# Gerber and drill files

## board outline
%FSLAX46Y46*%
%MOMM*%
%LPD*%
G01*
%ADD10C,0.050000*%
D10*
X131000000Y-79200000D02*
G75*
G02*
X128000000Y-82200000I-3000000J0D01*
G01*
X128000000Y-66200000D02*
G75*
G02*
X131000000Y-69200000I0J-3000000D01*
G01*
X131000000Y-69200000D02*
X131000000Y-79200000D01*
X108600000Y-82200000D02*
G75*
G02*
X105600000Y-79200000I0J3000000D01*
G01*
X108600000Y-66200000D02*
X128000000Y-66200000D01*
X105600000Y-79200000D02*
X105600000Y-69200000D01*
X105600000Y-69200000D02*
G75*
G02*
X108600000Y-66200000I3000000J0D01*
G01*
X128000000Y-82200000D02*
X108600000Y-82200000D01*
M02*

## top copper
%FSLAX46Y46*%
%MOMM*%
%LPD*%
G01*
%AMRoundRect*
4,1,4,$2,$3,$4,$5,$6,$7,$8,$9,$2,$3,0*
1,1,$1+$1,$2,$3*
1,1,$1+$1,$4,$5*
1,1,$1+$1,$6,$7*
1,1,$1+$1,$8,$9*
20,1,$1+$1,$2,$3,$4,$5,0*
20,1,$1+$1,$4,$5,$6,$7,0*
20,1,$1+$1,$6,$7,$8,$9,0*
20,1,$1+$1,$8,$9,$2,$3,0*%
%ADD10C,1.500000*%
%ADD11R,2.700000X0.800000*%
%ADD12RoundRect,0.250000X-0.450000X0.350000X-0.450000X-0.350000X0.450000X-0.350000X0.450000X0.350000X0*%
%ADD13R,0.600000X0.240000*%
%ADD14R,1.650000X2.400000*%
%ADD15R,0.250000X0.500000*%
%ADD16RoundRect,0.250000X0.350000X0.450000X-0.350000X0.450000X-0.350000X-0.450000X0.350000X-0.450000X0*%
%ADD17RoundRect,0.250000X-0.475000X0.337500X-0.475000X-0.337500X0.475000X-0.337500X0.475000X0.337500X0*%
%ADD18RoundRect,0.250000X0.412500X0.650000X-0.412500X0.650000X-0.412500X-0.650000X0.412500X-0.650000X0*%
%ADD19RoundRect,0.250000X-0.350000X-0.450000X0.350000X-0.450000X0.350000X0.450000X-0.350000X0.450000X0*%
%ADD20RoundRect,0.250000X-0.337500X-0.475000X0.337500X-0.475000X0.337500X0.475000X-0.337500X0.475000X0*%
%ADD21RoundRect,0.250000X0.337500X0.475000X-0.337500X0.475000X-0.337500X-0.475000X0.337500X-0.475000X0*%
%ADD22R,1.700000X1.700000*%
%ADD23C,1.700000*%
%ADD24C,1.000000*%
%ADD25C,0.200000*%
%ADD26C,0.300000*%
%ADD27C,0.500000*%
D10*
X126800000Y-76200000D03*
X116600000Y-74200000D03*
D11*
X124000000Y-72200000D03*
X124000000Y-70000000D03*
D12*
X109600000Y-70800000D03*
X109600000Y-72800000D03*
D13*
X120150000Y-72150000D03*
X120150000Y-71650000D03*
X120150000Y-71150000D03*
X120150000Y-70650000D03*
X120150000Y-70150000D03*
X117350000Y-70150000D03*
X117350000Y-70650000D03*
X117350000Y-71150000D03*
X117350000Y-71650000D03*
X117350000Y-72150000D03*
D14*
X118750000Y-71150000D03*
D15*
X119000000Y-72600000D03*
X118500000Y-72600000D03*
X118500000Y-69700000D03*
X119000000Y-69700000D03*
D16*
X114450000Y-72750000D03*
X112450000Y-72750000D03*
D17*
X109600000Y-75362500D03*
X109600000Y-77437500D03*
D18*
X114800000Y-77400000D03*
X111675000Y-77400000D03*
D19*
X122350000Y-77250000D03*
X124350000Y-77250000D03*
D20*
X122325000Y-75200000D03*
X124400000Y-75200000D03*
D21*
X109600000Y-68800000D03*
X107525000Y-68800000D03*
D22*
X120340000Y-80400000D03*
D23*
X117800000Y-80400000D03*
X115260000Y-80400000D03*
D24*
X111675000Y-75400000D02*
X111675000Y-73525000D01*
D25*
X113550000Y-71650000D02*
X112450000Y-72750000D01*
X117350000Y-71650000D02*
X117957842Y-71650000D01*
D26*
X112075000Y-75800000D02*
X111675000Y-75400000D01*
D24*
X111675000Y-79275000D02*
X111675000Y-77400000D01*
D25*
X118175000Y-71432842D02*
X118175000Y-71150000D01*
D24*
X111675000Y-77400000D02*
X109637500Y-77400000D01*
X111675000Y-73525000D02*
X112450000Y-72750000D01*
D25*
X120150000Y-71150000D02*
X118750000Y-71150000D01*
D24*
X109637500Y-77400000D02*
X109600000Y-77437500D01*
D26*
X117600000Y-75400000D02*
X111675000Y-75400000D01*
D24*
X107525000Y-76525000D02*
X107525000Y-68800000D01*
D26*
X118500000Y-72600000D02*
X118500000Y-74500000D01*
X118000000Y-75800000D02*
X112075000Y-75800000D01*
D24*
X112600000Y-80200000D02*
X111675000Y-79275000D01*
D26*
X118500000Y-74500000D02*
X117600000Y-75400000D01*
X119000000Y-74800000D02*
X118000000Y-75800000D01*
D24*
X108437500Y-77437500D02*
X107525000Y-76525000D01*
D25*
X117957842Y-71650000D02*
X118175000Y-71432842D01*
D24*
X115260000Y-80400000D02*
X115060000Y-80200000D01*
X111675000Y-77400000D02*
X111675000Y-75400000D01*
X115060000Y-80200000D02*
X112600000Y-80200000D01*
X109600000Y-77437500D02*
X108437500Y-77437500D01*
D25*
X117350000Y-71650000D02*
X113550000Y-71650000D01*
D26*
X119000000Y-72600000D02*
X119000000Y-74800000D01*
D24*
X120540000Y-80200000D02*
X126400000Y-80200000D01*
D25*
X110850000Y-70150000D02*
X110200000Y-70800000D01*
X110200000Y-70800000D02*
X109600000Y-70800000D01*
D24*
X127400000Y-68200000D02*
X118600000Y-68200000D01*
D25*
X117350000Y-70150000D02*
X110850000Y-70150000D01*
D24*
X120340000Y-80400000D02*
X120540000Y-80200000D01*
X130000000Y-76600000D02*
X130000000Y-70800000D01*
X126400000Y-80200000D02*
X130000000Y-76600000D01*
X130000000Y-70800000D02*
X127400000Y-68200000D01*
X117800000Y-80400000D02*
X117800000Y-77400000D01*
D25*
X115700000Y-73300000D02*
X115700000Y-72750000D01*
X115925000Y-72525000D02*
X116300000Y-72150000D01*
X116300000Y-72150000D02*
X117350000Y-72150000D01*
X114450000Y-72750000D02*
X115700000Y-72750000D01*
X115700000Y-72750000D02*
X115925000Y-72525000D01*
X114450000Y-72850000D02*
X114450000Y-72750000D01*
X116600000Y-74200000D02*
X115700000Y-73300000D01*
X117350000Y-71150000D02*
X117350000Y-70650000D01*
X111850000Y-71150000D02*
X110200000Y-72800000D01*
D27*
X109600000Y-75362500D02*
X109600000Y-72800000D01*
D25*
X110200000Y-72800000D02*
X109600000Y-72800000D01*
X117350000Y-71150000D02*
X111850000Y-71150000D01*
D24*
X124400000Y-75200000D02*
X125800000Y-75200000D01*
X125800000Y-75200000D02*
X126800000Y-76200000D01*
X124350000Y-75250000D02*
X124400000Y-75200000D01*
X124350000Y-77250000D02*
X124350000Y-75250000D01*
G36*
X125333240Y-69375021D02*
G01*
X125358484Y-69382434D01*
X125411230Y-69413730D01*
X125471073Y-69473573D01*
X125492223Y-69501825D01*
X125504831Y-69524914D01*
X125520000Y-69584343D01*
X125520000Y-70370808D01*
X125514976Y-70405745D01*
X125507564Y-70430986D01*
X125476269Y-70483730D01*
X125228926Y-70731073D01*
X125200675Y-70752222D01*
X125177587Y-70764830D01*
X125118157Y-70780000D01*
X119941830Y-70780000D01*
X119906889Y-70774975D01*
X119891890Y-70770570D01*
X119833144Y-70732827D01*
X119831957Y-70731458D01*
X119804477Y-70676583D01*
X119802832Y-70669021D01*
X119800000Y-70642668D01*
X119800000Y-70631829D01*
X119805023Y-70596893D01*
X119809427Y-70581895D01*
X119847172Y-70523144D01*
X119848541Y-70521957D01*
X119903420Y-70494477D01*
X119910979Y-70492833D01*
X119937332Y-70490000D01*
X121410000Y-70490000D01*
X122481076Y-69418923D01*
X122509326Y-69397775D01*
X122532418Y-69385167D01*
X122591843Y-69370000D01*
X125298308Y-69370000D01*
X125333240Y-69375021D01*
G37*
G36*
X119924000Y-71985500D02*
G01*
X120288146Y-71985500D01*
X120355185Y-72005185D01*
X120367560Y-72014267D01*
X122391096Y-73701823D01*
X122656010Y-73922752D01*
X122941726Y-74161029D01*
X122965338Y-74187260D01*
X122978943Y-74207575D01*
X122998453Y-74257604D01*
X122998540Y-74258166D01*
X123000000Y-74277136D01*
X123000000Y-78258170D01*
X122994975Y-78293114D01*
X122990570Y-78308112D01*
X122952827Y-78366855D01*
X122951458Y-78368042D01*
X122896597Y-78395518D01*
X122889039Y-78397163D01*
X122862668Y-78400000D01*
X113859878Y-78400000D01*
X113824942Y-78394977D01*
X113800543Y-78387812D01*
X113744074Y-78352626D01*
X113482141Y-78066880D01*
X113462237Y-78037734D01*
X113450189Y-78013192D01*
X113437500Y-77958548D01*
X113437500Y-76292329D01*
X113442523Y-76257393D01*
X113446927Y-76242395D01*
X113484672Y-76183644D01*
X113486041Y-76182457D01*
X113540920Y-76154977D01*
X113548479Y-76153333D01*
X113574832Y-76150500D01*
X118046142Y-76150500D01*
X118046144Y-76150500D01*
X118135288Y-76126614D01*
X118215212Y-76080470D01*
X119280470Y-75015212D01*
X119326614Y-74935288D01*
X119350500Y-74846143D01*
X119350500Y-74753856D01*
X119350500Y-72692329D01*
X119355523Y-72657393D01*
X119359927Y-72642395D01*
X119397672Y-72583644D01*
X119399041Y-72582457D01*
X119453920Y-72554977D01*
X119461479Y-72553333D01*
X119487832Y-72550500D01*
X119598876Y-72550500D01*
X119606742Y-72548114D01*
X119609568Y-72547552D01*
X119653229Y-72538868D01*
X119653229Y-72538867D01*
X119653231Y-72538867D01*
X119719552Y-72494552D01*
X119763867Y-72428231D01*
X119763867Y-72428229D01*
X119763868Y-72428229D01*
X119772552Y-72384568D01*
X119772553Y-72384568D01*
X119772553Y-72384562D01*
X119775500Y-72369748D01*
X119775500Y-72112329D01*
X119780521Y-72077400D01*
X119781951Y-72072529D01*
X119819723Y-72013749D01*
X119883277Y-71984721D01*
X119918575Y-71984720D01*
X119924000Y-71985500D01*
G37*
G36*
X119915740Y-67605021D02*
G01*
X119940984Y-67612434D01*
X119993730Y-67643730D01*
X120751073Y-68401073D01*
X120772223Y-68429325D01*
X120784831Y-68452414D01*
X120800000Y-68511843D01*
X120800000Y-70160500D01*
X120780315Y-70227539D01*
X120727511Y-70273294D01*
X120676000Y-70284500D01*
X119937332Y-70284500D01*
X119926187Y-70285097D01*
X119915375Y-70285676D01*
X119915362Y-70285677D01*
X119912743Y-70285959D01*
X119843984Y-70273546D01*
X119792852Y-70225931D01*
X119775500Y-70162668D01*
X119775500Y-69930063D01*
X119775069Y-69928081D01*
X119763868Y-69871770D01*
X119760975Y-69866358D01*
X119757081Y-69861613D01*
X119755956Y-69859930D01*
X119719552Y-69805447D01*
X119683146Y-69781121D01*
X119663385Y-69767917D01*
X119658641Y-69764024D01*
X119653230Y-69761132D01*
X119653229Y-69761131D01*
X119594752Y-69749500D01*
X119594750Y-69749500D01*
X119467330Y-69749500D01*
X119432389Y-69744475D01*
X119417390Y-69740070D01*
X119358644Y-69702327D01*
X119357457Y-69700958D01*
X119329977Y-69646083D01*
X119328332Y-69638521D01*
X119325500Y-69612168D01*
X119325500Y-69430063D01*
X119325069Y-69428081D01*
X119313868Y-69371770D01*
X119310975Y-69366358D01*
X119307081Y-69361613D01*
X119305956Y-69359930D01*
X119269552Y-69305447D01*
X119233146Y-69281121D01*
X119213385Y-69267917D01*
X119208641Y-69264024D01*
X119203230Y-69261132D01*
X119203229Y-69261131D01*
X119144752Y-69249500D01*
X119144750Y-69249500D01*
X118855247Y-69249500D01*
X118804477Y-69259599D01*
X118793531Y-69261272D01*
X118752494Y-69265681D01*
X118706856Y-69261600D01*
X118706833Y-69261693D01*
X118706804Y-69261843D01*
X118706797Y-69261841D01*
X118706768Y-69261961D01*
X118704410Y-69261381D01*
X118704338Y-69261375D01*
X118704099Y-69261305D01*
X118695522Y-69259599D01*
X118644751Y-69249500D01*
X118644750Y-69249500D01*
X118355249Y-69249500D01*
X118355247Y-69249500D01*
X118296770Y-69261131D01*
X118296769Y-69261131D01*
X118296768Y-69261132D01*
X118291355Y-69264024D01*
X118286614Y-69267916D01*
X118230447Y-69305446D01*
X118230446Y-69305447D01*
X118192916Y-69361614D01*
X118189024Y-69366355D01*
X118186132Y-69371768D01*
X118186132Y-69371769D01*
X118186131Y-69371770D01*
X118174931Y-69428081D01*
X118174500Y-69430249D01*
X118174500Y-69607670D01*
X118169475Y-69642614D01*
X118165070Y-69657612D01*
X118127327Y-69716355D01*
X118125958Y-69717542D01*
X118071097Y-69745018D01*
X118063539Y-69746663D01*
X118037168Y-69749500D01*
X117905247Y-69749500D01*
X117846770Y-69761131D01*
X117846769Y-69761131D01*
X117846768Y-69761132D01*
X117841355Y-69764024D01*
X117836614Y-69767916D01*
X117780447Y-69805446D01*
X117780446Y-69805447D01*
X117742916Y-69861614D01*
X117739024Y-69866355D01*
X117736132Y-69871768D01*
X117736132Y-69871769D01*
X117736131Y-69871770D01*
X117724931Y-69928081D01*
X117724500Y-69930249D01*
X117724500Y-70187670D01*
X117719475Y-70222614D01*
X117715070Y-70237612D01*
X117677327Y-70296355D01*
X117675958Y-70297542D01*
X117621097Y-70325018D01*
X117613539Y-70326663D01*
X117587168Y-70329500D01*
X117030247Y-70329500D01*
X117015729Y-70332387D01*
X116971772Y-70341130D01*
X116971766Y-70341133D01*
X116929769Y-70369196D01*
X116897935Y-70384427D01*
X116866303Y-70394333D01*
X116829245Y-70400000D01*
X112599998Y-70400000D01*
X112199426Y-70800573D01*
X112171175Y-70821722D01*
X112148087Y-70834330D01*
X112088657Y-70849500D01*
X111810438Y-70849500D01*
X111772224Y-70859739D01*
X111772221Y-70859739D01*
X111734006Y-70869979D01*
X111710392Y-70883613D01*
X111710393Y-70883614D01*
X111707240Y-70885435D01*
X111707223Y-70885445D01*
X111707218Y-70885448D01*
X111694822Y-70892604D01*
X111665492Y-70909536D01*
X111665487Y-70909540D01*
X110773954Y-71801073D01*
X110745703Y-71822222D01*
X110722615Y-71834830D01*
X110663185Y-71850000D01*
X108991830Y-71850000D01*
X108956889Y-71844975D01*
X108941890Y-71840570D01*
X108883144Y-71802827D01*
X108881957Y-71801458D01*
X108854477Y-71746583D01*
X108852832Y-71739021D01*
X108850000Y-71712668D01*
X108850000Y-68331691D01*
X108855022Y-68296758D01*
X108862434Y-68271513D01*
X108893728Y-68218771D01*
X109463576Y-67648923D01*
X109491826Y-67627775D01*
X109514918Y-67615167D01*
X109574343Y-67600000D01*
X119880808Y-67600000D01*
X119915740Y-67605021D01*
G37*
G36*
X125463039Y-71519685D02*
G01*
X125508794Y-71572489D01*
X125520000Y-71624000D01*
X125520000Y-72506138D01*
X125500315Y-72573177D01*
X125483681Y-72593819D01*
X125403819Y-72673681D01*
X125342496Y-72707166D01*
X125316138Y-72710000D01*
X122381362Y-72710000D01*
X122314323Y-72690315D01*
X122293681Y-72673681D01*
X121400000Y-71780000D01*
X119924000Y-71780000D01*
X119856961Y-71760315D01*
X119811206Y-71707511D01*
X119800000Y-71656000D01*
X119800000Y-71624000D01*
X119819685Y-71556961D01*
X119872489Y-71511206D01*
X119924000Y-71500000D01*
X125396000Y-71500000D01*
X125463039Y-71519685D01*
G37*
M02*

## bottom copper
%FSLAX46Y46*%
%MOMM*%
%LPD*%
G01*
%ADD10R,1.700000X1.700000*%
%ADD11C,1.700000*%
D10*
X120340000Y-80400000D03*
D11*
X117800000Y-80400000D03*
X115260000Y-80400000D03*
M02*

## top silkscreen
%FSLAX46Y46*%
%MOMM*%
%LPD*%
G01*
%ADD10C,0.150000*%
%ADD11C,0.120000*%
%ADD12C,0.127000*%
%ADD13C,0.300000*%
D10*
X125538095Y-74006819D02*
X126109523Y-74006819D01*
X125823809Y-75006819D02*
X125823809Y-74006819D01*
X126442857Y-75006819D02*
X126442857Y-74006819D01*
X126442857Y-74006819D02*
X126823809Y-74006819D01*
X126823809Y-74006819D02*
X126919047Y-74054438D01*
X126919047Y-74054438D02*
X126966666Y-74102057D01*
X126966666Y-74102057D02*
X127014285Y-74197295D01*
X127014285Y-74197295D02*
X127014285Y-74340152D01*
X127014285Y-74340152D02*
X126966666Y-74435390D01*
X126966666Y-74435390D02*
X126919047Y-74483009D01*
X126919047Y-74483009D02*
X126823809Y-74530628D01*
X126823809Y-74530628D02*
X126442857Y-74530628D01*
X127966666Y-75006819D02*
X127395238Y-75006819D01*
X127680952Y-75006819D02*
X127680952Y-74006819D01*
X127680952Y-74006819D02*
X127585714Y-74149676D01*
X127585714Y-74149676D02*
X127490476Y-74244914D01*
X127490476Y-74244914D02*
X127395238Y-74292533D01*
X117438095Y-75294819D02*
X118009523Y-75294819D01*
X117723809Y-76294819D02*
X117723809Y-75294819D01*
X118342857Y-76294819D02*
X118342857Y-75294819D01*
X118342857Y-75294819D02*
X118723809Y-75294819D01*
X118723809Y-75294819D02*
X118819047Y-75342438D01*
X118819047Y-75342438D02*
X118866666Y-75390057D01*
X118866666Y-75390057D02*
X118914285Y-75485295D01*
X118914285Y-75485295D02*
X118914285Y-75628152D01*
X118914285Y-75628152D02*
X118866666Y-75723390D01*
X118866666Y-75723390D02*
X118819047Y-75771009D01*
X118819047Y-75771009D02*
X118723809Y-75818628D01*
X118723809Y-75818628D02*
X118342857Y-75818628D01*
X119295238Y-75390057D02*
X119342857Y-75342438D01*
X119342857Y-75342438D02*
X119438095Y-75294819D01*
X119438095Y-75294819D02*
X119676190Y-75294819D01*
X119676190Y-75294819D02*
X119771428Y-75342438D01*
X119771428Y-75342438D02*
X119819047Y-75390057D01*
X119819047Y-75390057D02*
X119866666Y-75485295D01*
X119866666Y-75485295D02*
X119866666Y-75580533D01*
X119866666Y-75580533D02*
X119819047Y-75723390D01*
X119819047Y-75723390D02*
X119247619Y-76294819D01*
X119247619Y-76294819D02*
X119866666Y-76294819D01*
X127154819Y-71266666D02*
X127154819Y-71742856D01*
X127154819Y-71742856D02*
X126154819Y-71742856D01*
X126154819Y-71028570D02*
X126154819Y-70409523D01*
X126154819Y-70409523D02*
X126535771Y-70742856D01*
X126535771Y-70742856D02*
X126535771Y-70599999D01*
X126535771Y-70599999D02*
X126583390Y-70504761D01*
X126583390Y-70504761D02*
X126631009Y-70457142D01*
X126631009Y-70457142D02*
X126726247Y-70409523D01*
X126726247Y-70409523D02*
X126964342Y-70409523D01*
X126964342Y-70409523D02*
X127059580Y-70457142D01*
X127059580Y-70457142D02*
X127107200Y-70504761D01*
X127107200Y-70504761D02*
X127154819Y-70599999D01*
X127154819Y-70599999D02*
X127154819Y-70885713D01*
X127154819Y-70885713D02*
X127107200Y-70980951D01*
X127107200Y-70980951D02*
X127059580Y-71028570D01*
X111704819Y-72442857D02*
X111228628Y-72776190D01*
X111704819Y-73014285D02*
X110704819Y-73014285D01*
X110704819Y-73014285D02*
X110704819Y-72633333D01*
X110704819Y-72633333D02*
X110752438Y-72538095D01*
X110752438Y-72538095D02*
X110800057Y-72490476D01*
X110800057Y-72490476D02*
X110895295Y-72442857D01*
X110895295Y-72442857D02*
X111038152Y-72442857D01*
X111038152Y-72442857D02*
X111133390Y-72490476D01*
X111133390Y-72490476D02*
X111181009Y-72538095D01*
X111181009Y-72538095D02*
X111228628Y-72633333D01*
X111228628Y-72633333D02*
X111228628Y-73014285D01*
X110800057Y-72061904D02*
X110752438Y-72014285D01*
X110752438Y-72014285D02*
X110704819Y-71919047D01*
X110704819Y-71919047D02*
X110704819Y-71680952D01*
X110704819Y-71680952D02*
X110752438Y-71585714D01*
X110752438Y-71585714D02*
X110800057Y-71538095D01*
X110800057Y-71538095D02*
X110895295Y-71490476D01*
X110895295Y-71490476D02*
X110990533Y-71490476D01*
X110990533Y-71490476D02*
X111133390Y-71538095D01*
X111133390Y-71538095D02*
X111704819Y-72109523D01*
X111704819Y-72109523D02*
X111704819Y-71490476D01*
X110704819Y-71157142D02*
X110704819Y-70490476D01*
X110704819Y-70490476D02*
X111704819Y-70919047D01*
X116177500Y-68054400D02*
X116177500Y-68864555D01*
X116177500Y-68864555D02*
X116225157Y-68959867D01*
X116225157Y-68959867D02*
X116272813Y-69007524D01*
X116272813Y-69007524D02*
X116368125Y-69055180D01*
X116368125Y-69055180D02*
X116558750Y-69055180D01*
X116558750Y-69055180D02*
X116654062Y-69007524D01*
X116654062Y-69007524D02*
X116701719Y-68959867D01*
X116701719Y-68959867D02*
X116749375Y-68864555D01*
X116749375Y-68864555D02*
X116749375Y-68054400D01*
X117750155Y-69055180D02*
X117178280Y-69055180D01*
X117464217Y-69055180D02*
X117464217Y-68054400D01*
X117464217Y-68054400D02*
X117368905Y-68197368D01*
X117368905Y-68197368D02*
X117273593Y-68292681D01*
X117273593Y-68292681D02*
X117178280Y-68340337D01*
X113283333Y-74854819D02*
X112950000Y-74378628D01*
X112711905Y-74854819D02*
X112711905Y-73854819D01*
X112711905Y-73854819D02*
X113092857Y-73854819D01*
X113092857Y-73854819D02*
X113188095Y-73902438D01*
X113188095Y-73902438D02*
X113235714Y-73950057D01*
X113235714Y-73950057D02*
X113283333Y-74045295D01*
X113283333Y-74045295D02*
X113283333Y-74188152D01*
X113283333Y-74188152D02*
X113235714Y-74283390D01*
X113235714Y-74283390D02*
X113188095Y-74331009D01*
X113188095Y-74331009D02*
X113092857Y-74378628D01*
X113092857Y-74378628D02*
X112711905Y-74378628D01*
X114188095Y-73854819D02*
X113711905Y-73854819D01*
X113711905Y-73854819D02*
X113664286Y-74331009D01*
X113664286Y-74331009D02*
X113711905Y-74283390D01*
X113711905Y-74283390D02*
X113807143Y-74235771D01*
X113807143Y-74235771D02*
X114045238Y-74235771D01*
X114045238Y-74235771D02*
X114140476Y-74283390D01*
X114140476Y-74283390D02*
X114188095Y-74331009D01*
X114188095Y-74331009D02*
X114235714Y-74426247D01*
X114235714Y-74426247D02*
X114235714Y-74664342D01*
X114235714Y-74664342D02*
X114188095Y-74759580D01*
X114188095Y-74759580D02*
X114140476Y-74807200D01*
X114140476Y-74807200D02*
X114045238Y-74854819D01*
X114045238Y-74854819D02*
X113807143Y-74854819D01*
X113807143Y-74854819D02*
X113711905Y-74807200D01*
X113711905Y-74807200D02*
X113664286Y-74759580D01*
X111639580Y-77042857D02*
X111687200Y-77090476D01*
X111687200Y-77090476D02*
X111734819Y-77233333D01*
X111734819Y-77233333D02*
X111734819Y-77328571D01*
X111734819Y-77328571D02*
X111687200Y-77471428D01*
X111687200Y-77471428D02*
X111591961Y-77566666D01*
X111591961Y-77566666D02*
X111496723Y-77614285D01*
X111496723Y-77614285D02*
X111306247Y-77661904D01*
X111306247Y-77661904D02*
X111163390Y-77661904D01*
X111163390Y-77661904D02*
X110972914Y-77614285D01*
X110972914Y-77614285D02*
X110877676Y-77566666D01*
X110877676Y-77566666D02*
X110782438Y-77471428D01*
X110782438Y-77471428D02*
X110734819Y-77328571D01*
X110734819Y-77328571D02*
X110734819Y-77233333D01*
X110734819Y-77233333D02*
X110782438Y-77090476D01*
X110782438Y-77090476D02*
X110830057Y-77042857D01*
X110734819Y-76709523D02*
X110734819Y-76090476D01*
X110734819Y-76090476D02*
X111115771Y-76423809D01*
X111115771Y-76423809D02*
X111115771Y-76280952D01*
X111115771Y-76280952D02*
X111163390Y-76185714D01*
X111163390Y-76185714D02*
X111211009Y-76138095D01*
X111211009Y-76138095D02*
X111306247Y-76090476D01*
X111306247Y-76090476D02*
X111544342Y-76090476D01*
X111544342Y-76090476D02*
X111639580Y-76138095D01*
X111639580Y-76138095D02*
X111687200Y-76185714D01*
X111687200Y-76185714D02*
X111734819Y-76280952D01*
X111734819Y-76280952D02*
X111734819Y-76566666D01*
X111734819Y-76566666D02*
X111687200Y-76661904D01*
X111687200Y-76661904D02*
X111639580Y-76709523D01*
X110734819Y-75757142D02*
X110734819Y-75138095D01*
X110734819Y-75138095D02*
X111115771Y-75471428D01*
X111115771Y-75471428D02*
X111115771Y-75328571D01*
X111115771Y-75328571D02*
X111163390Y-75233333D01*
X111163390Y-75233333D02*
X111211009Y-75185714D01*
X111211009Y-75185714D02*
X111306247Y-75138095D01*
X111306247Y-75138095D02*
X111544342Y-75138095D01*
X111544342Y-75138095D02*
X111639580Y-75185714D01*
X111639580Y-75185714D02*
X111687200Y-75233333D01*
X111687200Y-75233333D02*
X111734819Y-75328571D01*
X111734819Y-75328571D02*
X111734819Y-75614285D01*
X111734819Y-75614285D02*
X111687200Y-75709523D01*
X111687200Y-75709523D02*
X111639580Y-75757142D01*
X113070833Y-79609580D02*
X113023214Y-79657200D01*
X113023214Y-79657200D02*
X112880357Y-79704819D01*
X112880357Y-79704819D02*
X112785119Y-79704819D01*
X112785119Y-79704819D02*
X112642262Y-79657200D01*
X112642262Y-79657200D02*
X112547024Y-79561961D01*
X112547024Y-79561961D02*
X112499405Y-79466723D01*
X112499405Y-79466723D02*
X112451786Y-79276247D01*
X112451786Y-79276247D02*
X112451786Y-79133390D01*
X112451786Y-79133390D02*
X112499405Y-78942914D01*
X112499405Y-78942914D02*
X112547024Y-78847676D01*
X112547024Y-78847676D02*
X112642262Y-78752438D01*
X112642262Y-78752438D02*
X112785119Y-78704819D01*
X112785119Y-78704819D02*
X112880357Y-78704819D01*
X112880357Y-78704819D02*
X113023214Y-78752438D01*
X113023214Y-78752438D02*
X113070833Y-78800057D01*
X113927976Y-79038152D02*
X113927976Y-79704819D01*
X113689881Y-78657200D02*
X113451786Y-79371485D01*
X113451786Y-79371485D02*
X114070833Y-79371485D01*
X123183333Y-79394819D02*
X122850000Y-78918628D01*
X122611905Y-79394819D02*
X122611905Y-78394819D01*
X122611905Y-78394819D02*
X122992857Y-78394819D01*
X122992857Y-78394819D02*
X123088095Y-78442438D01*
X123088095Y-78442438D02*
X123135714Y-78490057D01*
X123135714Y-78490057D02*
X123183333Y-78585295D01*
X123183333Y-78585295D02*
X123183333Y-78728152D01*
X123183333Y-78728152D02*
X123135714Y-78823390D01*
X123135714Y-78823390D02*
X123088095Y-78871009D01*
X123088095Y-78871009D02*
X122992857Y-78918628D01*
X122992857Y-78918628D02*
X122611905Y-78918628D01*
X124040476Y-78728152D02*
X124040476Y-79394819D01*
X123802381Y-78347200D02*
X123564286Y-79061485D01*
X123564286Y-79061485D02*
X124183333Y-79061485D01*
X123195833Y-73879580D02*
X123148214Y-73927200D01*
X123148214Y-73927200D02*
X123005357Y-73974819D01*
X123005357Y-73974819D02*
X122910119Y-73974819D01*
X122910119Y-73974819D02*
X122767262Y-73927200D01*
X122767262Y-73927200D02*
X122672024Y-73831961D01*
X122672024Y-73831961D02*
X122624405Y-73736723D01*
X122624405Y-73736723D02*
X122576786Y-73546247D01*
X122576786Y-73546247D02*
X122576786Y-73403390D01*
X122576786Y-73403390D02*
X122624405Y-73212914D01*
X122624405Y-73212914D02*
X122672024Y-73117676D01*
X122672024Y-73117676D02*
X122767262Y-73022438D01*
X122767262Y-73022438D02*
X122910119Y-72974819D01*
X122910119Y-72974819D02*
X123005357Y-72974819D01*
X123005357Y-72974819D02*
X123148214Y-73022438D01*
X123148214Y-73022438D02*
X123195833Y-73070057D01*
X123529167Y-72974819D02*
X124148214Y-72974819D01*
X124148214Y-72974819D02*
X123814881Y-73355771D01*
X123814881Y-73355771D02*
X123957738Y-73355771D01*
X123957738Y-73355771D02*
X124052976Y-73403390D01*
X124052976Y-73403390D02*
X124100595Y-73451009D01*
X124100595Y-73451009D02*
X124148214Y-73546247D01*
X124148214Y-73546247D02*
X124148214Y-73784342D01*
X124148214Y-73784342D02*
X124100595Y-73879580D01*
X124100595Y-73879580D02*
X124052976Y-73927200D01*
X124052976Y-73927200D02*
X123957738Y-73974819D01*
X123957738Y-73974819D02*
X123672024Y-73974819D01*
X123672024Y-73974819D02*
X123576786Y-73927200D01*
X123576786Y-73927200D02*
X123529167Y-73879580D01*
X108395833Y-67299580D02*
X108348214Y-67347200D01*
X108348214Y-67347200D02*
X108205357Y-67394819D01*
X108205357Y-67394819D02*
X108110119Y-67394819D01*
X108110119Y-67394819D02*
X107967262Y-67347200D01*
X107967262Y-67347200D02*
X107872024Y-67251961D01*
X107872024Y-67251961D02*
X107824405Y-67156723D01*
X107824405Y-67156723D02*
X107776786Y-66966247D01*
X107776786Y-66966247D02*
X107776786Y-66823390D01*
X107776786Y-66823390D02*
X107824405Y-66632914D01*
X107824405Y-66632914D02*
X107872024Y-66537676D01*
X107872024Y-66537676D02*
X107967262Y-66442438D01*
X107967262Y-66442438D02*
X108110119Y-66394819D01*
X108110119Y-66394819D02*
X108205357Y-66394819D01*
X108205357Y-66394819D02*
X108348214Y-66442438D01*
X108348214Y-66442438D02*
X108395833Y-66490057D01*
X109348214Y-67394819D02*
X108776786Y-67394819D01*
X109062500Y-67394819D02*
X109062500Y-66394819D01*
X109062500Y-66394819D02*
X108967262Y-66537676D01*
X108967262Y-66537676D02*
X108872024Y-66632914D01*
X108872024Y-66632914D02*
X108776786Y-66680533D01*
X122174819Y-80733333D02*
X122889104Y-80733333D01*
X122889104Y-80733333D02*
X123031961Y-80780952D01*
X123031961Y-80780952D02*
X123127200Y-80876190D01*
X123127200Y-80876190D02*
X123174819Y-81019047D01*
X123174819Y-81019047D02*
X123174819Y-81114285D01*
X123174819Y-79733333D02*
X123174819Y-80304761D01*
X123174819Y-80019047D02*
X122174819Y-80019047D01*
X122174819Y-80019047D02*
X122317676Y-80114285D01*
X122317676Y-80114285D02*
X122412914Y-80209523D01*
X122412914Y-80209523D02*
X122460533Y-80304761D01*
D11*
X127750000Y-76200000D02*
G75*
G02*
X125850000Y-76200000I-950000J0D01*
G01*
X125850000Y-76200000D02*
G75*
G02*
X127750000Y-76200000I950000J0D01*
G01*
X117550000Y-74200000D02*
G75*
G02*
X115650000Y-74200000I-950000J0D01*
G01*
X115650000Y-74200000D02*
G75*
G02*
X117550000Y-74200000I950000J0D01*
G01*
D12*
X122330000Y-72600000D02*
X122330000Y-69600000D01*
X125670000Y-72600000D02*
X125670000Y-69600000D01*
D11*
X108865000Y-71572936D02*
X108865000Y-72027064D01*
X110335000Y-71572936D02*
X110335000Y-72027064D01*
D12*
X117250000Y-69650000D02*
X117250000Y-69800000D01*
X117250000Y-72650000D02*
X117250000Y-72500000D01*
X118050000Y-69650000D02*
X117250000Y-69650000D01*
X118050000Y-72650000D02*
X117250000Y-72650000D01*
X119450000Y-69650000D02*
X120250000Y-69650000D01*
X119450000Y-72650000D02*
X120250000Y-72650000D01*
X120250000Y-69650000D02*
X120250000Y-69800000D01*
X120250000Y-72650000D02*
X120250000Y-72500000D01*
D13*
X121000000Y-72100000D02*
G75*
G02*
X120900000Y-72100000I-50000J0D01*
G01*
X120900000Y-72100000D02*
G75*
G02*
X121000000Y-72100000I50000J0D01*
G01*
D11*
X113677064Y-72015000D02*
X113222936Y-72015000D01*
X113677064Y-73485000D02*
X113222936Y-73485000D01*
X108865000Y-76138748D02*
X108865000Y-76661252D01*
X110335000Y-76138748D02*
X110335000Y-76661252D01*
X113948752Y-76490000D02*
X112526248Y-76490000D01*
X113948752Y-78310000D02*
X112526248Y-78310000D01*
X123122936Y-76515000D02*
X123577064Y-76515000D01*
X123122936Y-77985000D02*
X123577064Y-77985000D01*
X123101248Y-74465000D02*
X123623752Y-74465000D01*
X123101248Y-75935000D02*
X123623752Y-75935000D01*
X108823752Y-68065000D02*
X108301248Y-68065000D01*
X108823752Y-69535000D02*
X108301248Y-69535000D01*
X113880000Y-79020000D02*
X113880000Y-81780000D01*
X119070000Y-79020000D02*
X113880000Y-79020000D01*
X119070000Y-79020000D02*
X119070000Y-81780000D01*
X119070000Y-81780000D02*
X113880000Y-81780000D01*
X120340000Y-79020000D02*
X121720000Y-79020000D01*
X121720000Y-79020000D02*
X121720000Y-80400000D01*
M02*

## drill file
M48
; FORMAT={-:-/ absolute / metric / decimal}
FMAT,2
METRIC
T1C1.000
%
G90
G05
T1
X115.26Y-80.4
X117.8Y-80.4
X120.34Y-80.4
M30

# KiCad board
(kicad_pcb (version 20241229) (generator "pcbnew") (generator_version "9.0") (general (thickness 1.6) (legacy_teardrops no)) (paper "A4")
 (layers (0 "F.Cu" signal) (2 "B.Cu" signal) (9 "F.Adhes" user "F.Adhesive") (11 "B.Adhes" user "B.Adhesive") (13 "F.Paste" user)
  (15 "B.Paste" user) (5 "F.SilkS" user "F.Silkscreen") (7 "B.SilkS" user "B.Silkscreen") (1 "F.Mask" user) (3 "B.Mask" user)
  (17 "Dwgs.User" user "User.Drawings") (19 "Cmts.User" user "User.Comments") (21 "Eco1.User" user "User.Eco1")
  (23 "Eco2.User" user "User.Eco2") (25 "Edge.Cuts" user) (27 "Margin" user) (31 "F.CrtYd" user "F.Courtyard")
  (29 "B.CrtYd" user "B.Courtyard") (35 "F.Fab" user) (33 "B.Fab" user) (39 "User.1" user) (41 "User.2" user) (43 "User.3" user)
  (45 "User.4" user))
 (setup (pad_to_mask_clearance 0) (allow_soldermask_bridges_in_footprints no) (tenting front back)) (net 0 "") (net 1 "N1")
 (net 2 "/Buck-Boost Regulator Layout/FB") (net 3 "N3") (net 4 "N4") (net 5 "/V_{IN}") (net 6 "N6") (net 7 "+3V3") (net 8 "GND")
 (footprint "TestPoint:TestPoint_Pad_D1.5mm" (layer "F.Cu") (at 126.8 76.2)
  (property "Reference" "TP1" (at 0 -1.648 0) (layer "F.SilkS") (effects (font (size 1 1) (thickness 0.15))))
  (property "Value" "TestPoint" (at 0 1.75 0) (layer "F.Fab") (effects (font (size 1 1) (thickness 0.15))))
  (fp_circle (center 0 0) (end 0 0.95) (stroke (width 0.12) (type solid)) (fill no) (layer "F.SilkS"))
  (pad "1" smd circle (at 0 0) (size 1.5 1.5) (layers "F.Cu" "F.Mask") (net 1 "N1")))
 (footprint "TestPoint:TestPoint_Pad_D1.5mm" (layer "F.Cu") (at 116.6 74.2)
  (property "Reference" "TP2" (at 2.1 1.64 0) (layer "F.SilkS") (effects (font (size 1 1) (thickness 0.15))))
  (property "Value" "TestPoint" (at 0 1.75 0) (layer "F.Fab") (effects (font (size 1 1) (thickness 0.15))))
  (fp_circle (center 0 0) (end 0 0.95) (stroke (width 0.12) (type solid)) (fill no) (layer "F.SilkS"))
  (pad "1" smd circle (at 0 0) (size 1.5 1.5) (layers "F.Cu" "F.Mask") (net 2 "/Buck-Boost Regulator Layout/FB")))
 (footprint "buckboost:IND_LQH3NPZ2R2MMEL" (layer "F.Cu") (at 124 71.1 90)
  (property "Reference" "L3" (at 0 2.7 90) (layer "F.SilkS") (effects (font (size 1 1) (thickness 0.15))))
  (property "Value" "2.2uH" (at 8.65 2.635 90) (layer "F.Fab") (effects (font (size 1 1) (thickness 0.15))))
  (fp_line (start -1.5 -1.67) (end 1.5 -1.67) (stroke (width 0.127) (type solid)) (layer "F.SilkS"))
  (fp_line (start -1.5 1.67) (end 1.5 1.67) (stroke (width 0.127) (type solid)) (layer "F.SilkS"))
  (pad "1" smd rect (at -1.1 0 90) (size 0.8 2.7) (layers "F.Cu" "F.Mask" "F.Paste") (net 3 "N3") (solder_mask_margin 0.102))
  (pad "2" smd rect (at 1.1 0 90) (size 0.8 2.7) (layers "F.Cu" "F.Mask" "F.Paste") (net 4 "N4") (solder_mask_margin 0.102)))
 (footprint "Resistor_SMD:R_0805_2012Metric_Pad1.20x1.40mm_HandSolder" (layer "F.Cu") (at 109.6 71.8 -90)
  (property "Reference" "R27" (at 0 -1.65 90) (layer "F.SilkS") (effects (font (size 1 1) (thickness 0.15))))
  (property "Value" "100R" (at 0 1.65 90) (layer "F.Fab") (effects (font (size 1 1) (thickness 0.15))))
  (fp_line (start -0.227064 0.735) (end 0.227064 0.735) (stroke (width 0.12) (type solid)) (layer "F.SilkS"))
  (fp_line (start -0.227064 -0.735) (end 0.227064 -0.735) (stroke (width 0.12) (type solid)) (layer "F.SilkS"))
  (pad "1" smd roundrect (at -1 0 270) (size 1.2 1.4) (layers "F.Cu" "F.Mask" "F.Paste") (roundrect_rratio 0.208333) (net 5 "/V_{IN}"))
  (pad "2" smd roundrect (at 1 0 270) (size 1.2 1.4) (layers "F.Cu" "F.Mask" "F.Paste") (roundrect_rratio 0.208333) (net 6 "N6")))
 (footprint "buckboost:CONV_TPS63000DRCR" (layer "F.Cu") (at 118.75 71.15 180)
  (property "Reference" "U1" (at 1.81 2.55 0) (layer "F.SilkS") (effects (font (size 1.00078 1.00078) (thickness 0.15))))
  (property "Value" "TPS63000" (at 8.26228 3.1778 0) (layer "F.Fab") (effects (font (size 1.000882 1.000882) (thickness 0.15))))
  (fp_line (start 1.5 1.5) (end 1.5 1.35) (stroke (width 0.127) (type solid)) (layer "F.SilkS"))
  (fp_line (start 1.5 -1.5) (end 1.5 -1.35) (stroke (width 0.127) (type solid)) (layer "F.SilkS"))
  (fp_line (start 0.7 1.5) (end 1.5 1.5) (stroke (width 0.127) (type solid)) (layer "F.SilkS"))
  (fp_line (start 0.7 -1.5) (end 1.5 -1.5) (stroke (width 0.127) (type solid)) (layer "F.SilkS"))
  (fp_line (start -0.7 1.5) (end -1.5 1.5) (stroke (width 0.127) (type solid)) (layer "F.SilkS"))
  (fp_line (start -0.7 -1.5) (end -1.5 -1.5) (stroke (width 0.127) (type solid)) (layer "F.SilkS"))
  (fp_line (start -1.5 1.5) (end -1.5 1.35) (stroke (width 0.127) (type solid)) (layer "F.SilkS"))
  (fp_line (start -1.5 -1.5) (end -1.5 -1.35) (stroke (width 0.127) (type solid)) (layer "F.SilkS"))
  (fp_circle (center -2.2 -0.95) (end -2.15 -0.95) (stroke (width 0.3) (type solid)) (fill no) (layer "F.SilkS"))
  (pad "1" smd rect (at -1.4 -1 180) (size 0.6 0.24) (layers "F.Cu" "F.Mask" "F.Paste") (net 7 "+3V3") (solder_mask_margin 0.102))
  (pad "2" smd rect (at -1.4 -0.5 180) (size 0.6 0.24) (layers "F.Cu" "F.Mask" "F.Paste") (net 3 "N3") (solder_mask_margin 0.102))
  (pad "3" smd rect (at -1.4 0 180) (size 0.6 0.24) (layers "F.Cu" "F.Mask" "F.Paste") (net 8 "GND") (solder_mask_margin 0.102))
  (pad "4" smd rect (at -1.4 0.5 180) (size 0.6 0.24) (layers "F.Cu" "F.Mask" "F.Paste") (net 4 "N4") (solder_mask_margin 0.102))
  (pad "5" smd rect (at -1.4 1 180) (size 0.6 0.24) (layers "F.Cu" "F.Mask" "F.Paste") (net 5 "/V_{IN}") (solder_mask_margin 0.102))
  (pad "6" smd rect (at 1.4 1 180) (size 0.6 0.24) (layers "F.Cu" "F.Mask" "F.Paste") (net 5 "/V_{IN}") (solder_mask_margin 0.102))
  (pad "7" smd rect (at 1.4 0.5 180) (size 0.6 0.24) (layers "F.Cu" "F.Mask" "F.Paste") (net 6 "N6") (solder_mask_margin 0.102))
  (pad "8" smd rect (at 1.4 0 180) (size 0.6 0.24) (layers "F.Cu" "F.Mask" "F.Paste") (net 6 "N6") (solder_mask_margin 0.102))
  (pad "9" smd rect (at 1.4 -0.5 180) (size 0.6 0.24) (layers "F.Cu" "F.Mask" "F.Paste") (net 8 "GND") (solder_mask_margin 0.102))
  (pad "10" smd rect (at 1.4 -1 180) (size 0.6 0.24) (layers "F.Cu" "F.Mask" "F.Paste") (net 2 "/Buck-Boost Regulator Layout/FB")
   (solder_mask_margin 0.102))
  (pad "11" smd rect (at 0 0 180) (size 1.65 2.4) (layers "F.Cu" "F.Mask") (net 8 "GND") (solder_mask_margin 0.102))
  (pad "11_1" smd rect (at -0.25 -1.45 180) (size 0.25 0.5) (layers "F.Cu" "F.Mask") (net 8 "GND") (solder_mask_margin 0.102))
  (pad "11_2" smd rect (at 0.25 -1.45 180) (size 0.25 0.5) (layers "F.Cu" "F.Mask") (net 8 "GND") (solder_mask_margin 0.102))
  (pad "11_3" smd rect (at 0.25 1.45 180) (size 0.25 0.5) (layers "F.Cu" "F.Mask") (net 8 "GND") (solder_mask_margin 0.102))
  (pad "11_4" smd rect (at -0.25 1.45 180) (size 0.25 0.5) (layers "F.Cu" "F.Mask") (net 8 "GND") (solder_mask_margin 0.102)))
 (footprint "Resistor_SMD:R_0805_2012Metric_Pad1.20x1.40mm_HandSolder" (layer "F.Cu") (at 113.45 72.75 180)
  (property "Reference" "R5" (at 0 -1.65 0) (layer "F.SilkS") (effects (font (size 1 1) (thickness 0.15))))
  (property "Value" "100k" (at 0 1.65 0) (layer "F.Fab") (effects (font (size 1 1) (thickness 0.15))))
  (fp_line (start -0.227064 0.735) (end 0.227064 0.735) (stroke (width 0.12) (type solid)) (layer "F.SilkS"))
  (fp_line (start -0.227064 -0.735) (end 0.227064 -0.735) (stroke (width 0.12) (type solid)) (layer "F.SilkS"))
  (pad "1" smd roundrect (at -1 0 180) (size 1.2 1.4) (layers "F.Cu" "F.Mask" "F.Paste") (roundrect_rratio 0.208333)
   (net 2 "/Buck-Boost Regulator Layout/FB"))
  (pad "2" smd roundrect (at 1 0 180) (size 1.2 1.4) (layers "F.Cu" "F.Mask" "F.Paste") (roundrect_rratio 0.208333) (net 8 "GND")))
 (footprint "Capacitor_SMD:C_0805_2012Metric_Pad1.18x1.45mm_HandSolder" (layer "F.Cu") (at 109.6 76.4 -90)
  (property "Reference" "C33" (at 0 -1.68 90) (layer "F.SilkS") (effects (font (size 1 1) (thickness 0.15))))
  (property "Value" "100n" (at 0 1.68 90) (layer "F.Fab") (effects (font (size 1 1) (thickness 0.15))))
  (fp_line (start -0.261252 0.735) (end 0.261252 0.735) (stroke (width 0.12) (type solid)) (layer "F.SilkS"))
  (fp_line (start -0.261252 -0.735) (end 0.261252 -0.735) (stroke (width 0.12) (type solid)) (layer "F.SilkS"))
  (pad "1" smd roundrect (at -1.0375 0 270) (size 1.175 1.45) (layers "F.Cu" "F.Mask" "F.Paste") (roundrect_rratio 0.212766) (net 6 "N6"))
  (pad "2" smd roundrect (at 1.0375 0 270) (size 1.175 1.45) (layers "F.Cu" "F.Mask" "F.Paste") (roundrect_rratio 0.212766) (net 8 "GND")))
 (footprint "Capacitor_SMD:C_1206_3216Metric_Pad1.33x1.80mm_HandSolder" (layer "F.Cu") (at 113.2375 77.4 180)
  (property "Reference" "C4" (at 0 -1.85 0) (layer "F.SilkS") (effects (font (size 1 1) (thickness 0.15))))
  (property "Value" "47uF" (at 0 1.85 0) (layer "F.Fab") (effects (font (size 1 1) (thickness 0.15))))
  (fp_line (start -0.711252 0.91) (end 0.711252 0.91) (stroke (width 0.12) (type solid)) (layer "F.SilkS"))
  (fp_line (start -0.711252 -0.91) (end 0.711252 -0.91) (stroke (width 0.12) (type solid)) (layer "F.SilkS"))
  (pad "1" smd roundrect (at -1.5625 0 180) (size 1.325 1.8) (layers "F.Cu" "F.Mask" "F.Paste") (roundrect_rratio 0.188679) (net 7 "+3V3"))
  (pad "2" smd roundrect (at 1.5625 0 180) (size 1.325 1.8) (layers "F.Cu" "F.Mask" "F.Paste") (roundrect_rratio 0.188679) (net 8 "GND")))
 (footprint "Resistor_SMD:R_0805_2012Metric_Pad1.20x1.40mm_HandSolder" (layer "F.Cu") (at 123.35 77.25)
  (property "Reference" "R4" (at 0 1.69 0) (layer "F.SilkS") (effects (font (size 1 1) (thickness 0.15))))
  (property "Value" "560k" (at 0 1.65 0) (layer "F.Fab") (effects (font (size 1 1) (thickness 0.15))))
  (fp_line (start -0.227064 -0.735) (end 0.227064 -0.735) (stroke (width 0.12) (type solid)) (layer "F.SilkS"))
  (fp_line (start -0.227064 0.735) (end 0.227064 0.735) (stroke (width 0.12) (type solid)) (layer "F.SilkS"))
  (pad "1" smd roundrect (at -1 0) (size 1.2 1.4) (layers "F.Cu" "F.Mask" "F.Paste") (roundrect_rratio 0.208333) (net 7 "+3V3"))
  (pad "2" smd roundrect (at 1 0) (size 1.2 1.4) (layers "F.Cu" "F.Mask" "F.Paste") (roundrect_rratio 0.208333) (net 1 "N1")))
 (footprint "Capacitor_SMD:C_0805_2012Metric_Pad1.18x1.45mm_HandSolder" (layer "F.Cu") (at 123.3625 75.2)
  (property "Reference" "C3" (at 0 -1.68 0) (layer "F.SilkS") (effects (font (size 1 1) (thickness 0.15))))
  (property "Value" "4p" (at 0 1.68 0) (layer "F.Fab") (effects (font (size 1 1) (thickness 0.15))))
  (fp_line (start -0.261252 -0.735) (end 0.261252 -0.735) (stroke (width 0.12) (type solid)) (layer "F.SilkS"))
  (fp_line (start -0.261252 0.735) (end 0.261252 0.735) (stroke (width 0.12) (type solid)) (layer "F.SilkS"))
  (pad "1" smd roundrect (at -1.0375 0) (size 1.175 1.45) (layers "F.Cu" "F.Mask" "F.Paste") (roundrect_rratio 0.212766) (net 7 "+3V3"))
  (pad "2" smd roundrect (at 1.0375 0) (size 1.175 1.45) (layers "F.Cu" "F.Mask" "F.Paste") (roundrect_rratio 0.212766) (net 1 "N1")))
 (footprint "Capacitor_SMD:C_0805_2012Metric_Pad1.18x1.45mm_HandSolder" (layer "F.Cu") (at 108.5625 68.8 180)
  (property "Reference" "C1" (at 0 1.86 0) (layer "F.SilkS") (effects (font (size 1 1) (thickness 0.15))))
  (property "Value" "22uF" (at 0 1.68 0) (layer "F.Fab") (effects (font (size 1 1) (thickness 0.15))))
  (fp_line (start -0.261252 0.735) (end 0.261252 0.735) (stroke (width 0.12) (type solid)) (layer "F.SilkS"))
  (fp_line (start -0.261252 -0.735) (end 0.261252 -0.735) (stroke (width 0.12) (type solid)) (layer "F.SilkS"))
  (pad "1" smd roundrect (at -1.0375 0 180) (size 1.175 1.45) (layers "F.Cu" "F.Mask" "F.Paste") (roundrect_rratio 0.212766)
   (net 5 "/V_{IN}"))
  (pad "2" smd roundrect (at 1.0375 0 180) (size 1.175 1.45) (layers "F.Cu" "F.Mask" "F.Paste") (roundrect_rratio 0.212766) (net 8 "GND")))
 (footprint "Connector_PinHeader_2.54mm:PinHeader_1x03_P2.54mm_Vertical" (layer "F.Cu") (at 120.34 80.4 -90)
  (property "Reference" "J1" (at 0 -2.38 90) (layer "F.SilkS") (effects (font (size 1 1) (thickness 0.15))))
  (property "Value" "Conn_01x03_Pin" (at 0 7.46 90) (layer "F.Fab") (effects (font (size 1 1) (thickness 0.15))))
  (fp_line (start -1.38 6.46) (end 1.38 6.46) (stroke (width 0.12) (type solid)) (layer "F.SilkS"))
  (fp_line (start -1.38 1.27) (end -1.38 6.46) (stroke (width 0.12) (type solid)) (layer "F.SilkS"))
  (fp_line (start -1.38 1.27) (end 1.38 1.27) (stroke (width 0.12) (type solid)) (layer "F.SilkS"))
  (fp_line (start 1.38 1.27) (end 1.38 6.46) (stroke (width 0.12) (type solid)) (layer "F.SilkS"))
  (fp_line (start -1.38 0) (end -1.38 -1.38) (stroke (width 0.12) (type solid)) (layer "F.SilkS"))
  (fp_line (start -1.38 -1.38) (end 0 -1.38) (stroke (width 0.12) (type solid)) (layer "F.SilkS"))
  (pad "1" thru_hole rect (at 0 0 270) (size 1.7 1.7) (drill 1) (layers "*.Cu" "*.Mask") (remove_unused_layers no) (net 5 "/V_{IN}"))
  (pad "2" thru_hole circle (at 0 2.54 270) (size 1.7 1.7) (drill 1) (layers "*.Cu" "*.Mask") (remove_unused_layers no) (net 7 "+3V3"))
  (pad "3" thru_hole circle (at 0 5.08 270) (size 1.7 1.7) (drill 1) (layers "*.Cu" "*.Mask") (remove_unused_layers no) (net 8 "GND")))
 (gr_arc (start 131 79.2) (mid 130.12132 81.32132) (end 128 82.2) (stroke (width 0.05) (type default)) (layer "Edge.Cuts"))
 (gr_arc (start 128 66.2) (mid 130.12132 67.07868) (end 131 69.2) (stroke (width 0.05) (type default)) (layer "Edge.Cuts"))
 (gr_line (start 131 69.2) (end 131 79.2) (stroke (width 0.05) (type default)) (layer "Edge.Cuts"))
 (gr_arc (start 108.6 82.2) (mid 106.47868 81.32132) (end 105.6 79.2) (stroke (width 0.05) (type default)) (layer "Edge.Cuts"))
 (gr_line (start 108.6 66.2) (end 128 66.2) (stroke (width 0.05) (type default)) (layer "Edge.Cuts"))
 (gr_line (start 105.6 79.2) (end 105.6 69.2) (stroke (width 0.05) (type default)) (layer "Edge.Cuts"))
 (gr_arc (start 105.6 69.2) (mid 106.47868 67.07868) (end 108.6 66.2) (stroke (width 0.05) (type default)) (layer "Edge.Cuts"))
 (gr_line (start 128 82.2) (end 108.6 82.2) (stroke (width 0.05) (type default)) (layer "Edge.Cuts"))
 (segment (start 111.675 75.4) (end 111.675 73.525) (width 1) (layer "F.Cu") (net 8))
 (segment (start 113.55 71.65) (end 112.45 72.75) (width 0.2) (layer "F.Cu") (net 8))
 (segment (start 117.35 71.65) (end 117.957842 71.65) (width 0.2) (layer "F.Cu") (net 8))
 (segment (start 112.075 75.8) (end 111.675 75.4) (width 0.3) (layer "F.Cu") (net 8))
 (segment (start 111.675 79.275) (end 111.675 77.4) (width 1) (layer "F.Cu") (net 8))
 (segment (start 118.175 71.432842) (end 118.175 71.15) (width 0.2) (layer "F.Cu") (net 8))
 (segment (start 111.675 77.4) (end 109.6375 77.4) (width 1) (layer "F.Cu") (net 8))
 (segment (start 111.675 73.525) (end 112.45 72.75) (width 1) (layer "F.Cu") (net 8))
 (segment (start 120.15 71.15) (end 118.75 71.15) (width 0.2) (layer "F.Cu") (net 8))
 (segment (start 109.6375 77.4) (end 109.6 77.4375) (width 1) (layer "F.Cu") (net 8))
 (segment (start 117.6 75.4) (end 111.675 75.4) (width 0.3) (layer "F.Cu") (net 8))
 (segment (start 107.525 76.525) (end 107.525 68.8) (width 1) (layer "F.Cu") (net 8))
 (segment (start 118.5 72.6) (end 118.5 74.5) (width 0.3) (layer "F.Cu") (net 8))
 (segment (start 118 75.8) (end 112.075 75.8) (width 0.3) (layer "F.Cu") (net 8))
 (segment (start 112.6 80.2) (end 111.675 79.275) (width 1) (layer "F.Cu") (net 8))
 (segment (start 118.5 74.5) (end 117.6 75.4) (width 0.3) (layer "F.Cu") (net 8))
 (segment (start 119 74.8) (end 118 75.8) (width 0.3) (layer "F.Cu") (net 8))
 (segment (start 108.4375 77.4375) (end 107.525 76.525) (width 1) (layer "F.Cu") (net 8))
 (segment (start 117.957842 71.65) (end 118.175 71.432842) (width 0.2) (layer "F.Cu") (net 8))
 (segment (start 115.26 80.4) (end 115.06 80.2) (width 1) (layer "F.Cu") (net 8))
 (segment (start 111.675 77.4) (end 111.675 75.4) (width 1) (layer "F.Cu") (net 8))
 (segment (start 115.06 80.2) (end 112.6 80.2) (width 1) (layer "F.Cu") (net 8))
 (segment (start 109.6 77.4375) (end 108.4375 77.4375) (width 1) (layer "F.Cu") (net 8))
 (segment (start 117.35 71.65) (end 113.55 71.65) (width 0.2) (layer "F.Cu") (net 8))
 (segment (start 119 72.6) (end 119 74.8) (width 0.3) (layer "F.Cu") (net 8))
 (segment (start 120.54 80.2) (end 126.4 80.2) (width 1) (layer "F.Cu") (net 5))
 (segment (start 110.85 70.15) (end 110.2 70.8) (width 0.2) (layer "F.Cu") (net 5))
 (segment (start 110.2 70.8) (end 109.6 70.8) (width 0.2) (layer "F.Cu") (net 5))
 (segment (start 127.4 68.2) (end 118.6 68.2) (width 1) (layer "F.Cu") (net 5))
 (segment (start 117.35 70.15) (end 110.85 70.15) (width 0.2) (layer "F.Cu") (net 5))
 (segment (start 120.34 80.4) (end 120.54 80.2) (width 1) (layer "F.Cu") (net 5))
 (segment (start 130 76.6) (end 130 70.8) (width 1) (layer "F.Cu") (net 5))
 (segment (start 126.4 80.2) (end 130 76.6) (width 1) (layer "F.Cu") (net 5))
 (segment (start 130 70.8) (end 127.4 68.2) (width 1) (layer "F.Cu") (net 5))
 (segment (start 117.8 80.4) (end 117.8 77.4) (width 1) (layer "F.Cu") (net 7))
 (segment (start 115.7 73.3) (end 115.7 72.75) (width 0.2) (layer "F.Cu") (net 2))
 (segment (start 115.925 72.525) (end 116.3 72.15) (width 0.2) (layer "F.Cu") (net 2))
 (segment (start 116.3 72.15) (end 117.35 72.15) (width 0.2) (layer "F.Cu") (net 2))
 (segment (start 114.45 72.75) (end 115.7 72.75) (width 0.2) (layer "F.Cu") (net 2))
 (segment (start 115.7 72.75) (end 115.925 72.525) (width 0.2) (layer "F.Cu") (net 2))
 (segment (start 114.45 72.85) (end 114.45 72.75) (width 0.2) (layer "F.Cu") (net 2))
 (segment (start 116.6 74.2) (end 115.7 73.3) (width 0.2) (layer "F.Cu") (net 2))
 (segment (start 117.35 71.15) (end 117.35 70.65) (width 0.2) (layer "F.Cu") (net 6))
 (segment (start 111.85 71.15) (end 110.2 72.8) (width 0.2) (layer "F.Cu") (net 6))
 (segment (start 109.6 75.3625) (end 109.6 72.8) (width 0.5) (layer "F.Cu") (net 6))
 (segment (start 110.2 72.8) (end 109.6 72.8) (width 0.2) (layer "F.Cu") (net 6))
 (segment (start 117.35 71.15) (end 111.85 71.15) (width 0.2) (layer "F.Cu") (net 6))
 (segment (start 124.4 75.2) (end 125.8 75.2) (width 1) (layer "F.Cu") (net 1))
 (segment (start 125.8 75.2) (end 126.8 76.2) (width 1) (layer "F.Cu") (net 1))
 (segment (start 124.35 75.25) (end 124.4 75.2) (width 1) (layer "F.Cu") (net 1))
 (segment (start 124.35 77.25) (end 124.35 75.25) (width 1) (layer "F.Cu") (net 1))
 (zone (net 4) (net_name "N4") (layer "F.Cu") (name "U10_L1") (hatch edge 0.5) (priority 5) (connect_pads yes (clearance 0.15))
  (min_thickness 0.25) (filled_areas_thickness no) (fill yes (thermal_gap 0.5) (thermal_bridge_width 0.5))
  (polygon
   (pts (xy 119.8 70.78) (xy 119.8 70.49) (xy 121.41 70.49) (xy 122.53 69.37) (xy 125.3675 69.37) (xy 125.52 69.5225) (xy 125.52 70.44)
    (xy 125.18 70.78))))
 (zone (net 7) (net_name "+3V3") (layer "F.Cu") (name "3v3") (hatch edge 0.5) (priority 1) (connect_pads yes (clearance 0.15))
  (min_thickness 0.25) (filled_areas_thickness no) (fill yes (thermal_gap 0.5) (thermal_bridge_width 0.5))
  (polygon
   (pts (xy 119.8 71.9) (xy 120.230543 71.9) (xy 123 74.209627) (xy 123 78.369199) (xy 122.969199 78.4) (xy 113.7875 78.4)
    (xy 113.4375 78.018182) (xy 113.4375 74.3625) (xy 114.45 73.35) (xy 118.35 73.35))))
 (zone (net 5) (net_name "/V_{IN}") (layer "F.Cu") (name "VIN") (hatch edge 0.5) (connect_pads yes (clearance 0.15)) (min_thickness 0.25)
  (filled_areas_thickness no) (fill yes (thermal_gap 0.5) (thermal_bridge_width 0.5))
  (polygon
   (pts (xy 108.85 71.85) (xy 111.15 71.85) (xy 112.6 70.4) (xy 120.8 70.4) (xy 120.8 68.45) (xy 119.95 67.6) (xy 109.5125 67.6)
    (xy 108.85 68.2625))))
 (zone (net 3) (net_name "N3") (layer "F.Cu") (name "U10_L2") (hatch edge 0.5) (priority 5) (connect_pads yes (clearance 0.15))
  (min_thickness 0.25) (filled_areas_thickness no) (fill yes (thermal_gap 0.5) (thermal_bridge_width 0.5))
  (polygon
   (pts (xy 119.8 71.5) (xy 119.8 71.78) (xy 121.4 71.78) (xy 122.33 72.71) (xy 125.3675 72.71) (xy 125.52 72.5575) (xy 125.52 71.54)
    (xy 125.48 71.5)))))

